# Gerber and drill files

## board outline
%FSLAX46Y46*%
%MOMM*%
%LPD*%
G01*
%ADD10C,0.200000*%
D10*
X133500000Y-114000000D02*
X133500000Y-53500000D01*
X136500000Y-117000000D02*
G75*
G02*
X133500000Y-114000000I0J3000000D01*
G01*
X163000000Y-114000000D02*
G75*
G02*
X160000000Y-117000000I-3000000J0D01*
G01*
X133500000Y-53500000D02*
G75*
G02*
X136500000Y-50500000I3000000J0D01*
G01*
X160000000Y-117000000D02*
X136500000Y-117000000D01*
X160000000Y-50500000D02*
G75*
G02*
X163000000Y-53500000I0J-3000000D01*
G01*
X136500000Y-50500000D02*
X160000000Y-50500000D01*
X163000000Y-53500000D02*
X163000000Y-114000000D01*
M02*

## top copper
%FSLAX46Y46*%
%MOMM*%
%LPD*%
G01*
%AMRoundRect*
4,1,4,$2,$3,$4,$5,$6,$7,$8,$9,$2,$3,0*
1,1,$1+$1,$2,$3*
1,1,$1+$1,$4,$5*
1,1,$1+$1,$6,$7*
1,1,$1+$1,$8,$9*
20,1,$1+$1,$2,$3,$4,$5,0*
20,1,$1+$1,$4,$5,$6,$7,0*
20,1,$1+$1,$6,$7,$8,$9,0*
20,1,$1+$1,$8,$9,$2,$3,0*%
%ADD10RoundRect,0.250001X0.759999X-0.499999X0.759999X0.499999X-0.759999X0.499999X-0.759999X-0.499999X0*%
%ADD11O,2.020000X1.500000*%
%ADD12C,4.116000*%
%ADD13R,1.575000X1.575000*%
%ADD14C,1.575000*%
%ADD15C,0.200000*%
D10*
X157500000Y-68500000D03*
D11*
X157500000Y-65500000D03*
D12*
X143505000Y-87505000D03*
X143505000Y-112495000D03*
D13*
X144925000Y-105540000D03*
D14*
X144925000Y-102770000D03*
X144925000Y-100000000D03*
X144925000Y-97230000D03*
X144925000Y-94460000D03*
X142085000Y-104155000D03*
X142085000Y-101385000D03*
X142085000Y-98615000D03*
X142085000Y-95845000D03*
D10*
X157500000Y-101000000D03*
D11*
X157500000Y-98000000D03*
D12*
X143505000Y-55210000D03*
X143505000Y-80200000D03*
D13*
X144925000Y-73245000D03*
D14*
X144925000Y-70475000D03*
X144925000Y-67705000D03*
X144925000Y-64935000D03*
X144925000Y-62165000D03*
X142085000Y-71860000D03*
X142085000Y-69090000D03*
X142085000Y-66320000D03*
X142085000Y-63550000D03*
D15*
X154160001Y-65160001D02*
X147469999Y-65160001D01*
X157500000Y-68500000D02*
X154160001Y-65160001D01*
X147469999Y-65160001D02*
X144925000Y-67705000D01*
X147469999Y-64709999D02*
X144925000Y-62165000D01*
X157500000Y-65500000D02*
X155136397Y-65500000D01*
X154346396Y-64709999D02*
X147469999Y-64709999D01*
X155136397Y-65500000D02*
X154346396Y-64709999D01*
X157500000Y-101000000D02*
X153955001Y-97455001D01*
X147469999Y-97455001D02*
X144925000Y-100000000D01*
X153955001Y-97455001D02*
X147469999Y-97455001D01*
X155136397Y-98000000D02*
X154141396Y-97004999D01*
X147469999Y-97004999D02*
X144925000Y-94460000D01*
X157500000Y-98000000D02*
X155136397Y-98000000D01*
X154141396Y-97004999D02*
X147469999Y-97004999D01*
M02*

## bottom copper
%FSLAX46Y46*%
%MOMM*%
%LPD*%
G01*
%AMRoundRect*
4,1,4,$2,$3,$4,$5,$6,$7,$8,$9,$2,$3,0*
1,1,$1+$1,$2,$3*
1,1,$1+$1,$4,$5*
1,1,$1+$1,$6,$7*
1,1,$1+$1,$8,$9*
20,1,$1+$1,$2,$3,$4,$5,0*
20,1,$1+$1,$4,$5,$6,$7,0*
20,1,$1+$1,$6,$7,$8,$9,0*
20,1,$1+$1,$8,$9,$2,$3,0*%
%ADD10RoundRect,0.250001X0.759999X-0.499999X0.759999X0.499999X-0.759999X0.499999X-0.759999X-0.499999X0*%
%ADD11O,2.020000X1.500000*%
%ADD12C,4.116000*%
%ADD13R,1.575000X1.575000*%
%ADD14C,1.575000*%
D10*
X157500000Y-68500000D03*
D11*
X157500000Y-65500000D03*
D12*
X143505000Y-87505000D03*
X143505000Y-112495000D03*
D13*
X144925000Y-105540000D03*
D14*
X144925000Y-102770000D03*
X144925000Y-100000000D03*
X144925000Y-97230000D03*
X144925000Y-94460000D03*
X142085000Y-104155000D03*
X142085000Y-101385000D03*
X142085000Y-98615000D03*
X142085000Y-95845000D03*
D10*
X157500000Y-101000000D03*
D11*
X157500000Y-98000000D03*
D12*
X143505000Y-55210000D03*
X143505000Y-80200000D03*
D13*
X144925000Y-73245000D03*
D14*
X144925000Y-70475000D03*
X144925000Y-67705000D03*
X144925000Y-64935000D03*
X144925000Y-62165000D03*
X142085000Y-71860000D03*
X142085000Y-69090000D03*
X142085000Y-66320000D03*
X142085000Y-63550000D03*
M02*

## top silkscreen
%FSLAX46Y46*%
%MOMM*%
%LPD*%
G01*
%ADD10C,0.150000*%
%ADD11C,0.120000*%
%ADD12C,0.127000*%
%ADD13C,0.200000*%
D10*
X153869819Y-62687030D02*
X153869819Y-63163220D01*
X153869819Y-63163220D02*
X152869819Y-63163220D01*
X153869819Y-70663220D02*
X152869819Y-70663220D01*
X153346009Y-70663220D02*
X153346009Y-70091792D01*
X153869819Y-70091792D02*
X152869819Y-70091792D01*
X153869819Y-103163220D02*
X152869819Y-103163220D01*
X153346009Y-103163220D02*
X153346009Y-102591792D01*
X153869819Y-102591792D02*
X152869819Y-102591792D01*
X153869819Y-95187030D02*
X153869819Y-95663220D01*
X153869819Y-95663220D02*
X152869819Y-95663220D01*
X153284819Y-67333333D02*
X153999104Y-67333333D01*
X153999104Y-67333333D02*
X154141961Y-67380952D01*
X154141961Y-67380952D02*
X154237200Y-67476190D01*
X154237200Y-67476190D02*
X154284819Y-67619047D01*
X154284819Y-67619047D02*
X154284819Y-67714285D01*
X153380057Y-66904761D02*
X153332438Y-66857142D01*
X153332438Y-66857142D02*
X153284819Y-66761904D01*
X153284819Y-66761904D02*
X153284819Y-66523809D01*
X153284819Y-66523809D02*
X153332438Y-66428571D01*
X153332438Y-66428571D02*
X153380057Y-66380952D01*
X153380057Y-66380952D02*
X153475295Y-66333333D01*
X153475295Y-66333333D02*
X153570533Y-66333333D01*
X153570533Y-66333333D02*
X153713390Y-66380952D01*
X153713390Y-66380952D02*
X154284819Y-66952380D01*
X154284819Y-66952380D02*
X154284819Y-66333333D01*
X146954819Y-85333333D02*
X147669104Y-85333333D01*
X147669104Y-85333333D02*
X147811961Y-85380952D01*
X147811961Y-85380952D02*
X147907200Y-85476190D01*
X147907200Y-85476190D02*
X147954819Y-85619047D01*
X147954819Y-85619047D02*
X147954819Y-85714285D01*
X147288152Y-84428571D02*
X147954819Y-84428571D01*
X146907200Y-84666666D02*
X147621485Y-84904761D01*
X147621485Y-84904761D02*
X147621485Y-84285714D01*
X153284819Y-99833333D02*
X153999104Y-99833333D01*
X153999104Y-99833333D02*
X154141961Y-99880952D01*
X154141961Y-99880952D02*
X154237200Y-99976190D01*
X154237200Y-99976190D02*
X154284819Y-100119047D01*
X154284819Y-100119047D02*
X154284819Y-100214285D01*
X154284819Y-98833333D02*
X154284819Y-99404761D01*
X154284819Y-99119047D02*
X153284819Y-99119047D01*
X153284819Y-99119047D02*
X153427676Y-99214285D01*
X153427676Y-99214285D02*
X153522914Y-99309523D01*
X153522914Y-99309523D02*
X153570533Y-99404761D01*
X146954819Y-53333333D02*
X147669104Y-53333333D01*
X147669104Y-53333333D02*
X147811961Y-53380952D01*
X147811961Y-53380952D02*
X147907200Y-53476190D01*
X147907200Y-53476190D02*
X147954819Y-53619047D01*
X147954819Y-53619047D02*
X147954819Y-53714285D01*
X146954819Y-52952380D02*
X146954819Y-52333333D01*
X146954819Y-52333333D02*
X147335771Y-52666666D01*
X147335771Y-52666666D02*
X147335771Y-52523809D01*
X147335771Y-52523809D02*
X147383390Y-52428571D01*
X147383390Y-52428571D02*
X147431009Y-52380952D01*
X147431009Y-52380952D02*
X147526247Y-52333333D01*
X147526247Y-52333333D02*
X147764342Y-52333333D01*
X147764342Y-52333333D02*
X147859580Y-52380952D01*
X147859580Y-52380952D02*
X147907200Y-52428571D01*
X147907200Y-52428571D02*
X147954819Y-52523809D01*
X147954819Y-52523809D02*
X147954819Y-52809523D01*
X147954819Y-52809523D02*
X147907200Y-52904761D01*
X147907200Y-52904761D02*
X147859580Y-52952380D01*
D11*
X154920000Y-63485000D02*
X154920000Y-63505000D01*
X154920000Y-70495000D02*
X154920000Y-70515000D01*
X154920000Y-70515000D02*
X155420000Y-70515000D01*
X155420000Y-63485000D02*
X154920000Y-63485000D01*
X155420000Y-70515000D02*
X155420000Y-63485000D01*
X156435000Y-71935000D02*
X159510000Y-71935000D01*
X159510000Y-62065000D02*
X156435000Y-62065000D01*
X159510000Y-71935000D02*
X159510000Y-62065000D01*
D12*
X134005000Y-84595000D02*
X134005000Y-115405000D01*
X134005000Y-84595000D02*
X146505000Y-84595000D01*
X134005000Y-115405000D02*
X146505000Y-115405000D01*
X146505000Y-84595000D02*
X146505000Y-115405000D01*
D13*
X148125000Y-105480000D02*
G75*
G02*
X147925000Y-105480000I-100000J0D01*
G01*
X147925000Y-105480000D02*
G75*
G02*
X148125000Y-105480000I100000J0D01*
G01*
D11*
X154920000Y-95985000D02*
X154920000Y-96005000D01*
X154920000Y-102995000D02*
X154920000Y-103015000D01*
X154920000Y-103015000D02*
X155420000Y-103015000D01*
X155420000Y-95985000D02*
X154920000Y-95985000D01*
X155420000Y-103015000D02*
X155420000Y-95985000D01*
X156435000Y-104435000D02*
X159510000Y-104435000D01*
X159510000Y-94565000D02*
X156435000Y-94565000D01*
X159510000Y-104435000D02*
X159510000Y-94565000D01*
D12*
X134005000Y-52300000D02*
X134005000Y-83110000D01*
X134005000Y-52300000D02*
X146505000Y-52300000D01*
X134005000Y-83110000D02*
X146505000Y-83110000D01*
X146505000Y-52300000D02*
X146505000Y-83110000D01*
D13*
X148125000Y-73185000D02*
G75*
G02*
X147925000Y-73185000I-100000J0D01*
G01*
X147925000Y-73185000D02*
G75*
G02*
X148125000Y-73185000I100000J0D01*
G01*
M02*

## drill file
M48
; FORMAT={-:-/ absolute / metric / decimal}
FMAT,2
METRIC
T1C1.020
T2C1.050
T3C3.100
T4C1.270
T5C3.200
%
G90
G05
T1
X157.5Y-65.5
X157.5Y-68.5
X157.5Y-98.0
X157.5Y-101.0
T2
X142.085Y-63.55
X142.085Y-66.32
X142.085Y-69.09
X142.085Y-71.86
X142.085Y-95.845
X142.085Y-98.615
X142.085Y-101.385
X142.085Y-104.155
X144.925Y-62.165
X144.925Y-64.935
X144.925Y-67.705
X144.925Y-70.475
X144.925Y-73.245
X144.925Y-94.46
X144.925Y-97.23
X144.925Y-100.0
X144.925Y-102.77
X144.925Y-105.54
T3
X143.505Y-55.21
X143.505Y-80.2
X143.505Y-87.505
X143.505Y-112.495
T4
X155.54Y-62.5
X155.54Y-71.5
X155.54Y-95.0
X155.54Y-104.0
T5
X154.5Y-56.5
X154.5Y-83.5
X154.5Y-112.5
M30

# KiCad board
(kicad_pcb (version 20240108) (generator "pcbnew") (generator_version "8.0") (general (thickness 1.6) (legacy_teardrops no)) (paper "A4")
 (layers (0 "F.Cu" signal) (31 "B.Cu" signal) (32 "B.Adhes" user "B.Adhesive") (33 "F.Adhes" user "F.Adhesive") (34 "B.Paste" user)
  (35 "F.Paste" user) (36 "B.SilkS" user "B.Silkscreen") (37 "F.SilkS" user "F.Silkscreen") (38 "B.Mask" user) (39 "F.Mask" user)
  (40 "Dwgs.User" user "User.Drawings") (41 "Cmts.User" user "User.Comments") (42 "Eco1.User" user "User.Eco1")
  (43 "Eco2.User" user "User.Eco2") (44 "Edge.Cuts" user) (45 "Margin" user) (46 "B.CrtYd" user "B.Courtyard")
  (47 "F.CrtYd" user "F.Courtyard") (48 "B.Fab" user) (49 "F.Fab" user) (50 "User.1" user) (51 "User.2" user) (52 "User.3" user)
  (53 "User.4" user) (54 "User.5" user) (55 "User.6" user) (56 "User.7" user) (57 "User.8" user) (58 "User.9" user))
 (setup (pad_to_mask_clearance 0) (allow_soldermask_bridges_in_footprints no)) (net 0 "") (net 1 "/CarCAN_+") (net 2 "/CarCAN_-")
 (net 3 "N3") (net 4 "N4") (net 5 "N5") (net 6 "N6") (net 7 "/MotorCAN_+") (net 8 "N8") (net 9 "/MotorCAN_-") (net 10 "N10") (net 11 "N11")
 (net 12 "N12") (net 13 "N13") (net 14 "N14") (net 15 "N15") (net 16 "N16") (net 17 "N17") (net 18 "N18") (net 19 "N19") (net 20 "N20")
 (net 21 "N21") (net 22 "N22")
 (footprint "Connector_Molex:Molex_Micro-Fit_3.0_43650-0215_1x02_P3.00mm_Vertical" (layer "F.Cu") (at 157.5 68.5 90)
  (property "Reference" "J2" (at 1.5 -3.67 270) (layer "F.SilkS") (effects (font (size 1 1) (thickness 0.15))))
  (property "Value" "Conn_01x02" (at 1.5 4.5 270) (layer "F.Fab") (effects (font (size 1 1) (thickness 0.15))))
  (fp_line (start 5.015 -2.58) (end 4.995 -2.58) (stroke (width 0.12) (type solid)) (layer "F.SilkS"))
  (fp_line (start -1.995 -2.58) (end -2.015 -2.58) (stroke (width 0.12) (type solid)) (layer "F.SilkS"))
  (fp_line (start -2.015 -2.58) (end -2.015 -2.08) (stroke (width 0.12) (type solid)) (layer "F.SilkS"))
  (fp_line (start 5.015 -2.08) (end 5.015 -2.58) (stroke (width 0.12) (type solid)) (layer "F.SilkS"))
  (fp_line (start -2.015 -2.08) (end 5.015 -2.08) (stroke (width 0.12) (type solid)) (layer "F.SilkS"))
  (fp_line (start -3.435 -1.065) (end -3.435 2.01) (stroke (width 0.12) (type solid)) (layer "F.SilkS"))
  (fp_line (start 6.435 2.01) (end 6.435 -1.065) (stroke (width 0.12) (type solid)) (layer "F.SilkS"))
  (fp_line (start -3.435 2.01) (end 6.435 2.01) (stroke (width 0.12) (type solid)) (layer "F.SilkS"))
  (pad "" np_thru_hole circle (at -3 -1.96 90) (size 1.27 1.27) (drill 1.27) (layers "*.Cu" "*.Mask"))
  (pad "" np_thru_hole circle (at 6 -1.96 90) (size 1.27 1.27) (drill 1.27) (layers "*.Cu" "*.Mask"))
  (pad "1" thru_hole roundrect (at 0 0 90) (size 1.5 2.02) (drill 1.02) (layers "*.Cu" "*.Mask") (remove_unused_layers no)
   (roundrect_rratio 0.166667) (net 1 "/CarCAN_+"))
  (pad "2" thru_hole oval (at 3 0 90) (size 1.5 2.02) (drill 1.02) (layers "*.Cu" "*.Mask") (remove_unused_layers no) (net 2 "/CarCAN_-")))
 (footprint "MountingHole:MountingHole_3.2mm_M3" (layer "F.Cu") (at 154.5 112.5)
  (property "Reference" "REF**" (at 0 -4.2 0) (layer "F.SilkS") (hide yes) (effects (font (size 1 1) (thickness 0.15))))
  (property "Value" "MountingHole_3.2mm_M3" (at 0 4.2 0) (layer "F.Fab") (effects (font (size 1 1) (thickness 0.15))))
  (pad "" np_thru_hole circle (at 0 0) (size 3.2 3.2) (drill 3.2) (layers "F&B.Cu" "*.Mask")))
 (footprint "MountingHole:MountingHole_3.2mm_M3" (layer "F.Cu") (at 154.5 56.5)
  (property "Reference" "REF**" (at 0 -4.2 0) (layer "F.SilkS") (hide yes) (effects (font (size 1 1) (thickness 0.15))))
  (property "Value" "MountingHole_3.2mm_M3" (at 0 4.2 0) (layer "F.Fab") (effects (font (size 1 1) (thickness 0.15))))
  (pad "" np_thru_hole circle (at 0 0) (size 3.2 3.2) (drill 3.2) (layers "*.Cu" "*.Mask")))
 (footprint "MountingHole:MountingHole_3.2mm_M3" (layer "F.Cu") (at 154.5 83.5)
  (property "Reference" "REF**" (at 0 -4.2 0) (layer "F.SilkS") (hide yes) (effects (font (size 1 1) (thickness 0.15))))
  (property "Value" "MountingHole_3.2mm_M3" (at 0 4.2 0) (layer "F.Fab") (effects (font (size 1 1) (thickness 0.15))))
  (pad "" np_thru_hole circle (at 0 0) (size 3.2 3.2) (drill 3.2) (layers "F&B.Cu" "*.Mask")))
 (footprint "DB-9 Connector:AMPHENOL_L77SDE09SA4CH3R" (layer "F.Cu") (at 143.505 100 -90)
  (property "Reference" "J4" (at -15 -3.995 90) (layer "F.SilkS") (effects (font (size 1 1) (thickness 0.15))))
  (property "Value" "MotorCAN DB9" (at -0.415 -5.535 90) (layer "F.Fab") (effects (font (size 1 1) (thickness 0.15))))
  (fp_line (start -15.405 9.5) (end 15.405 9.5) (stroke (width 0.127) (type solid)) (layer "F.SilkS"))
  (fp_line (start -15.405 9.5) (end -15.405 -3) (stroke (width 0.127) (type solid)) (layer "F.SilkS"))
  (fp_line (start 15.405 9.5) (end 15.405 -3) (stroke (width 0.127) (type solid)) (layer "F.SilkS"))
  (fp_line (start -15.405 -3) (end 15.405 -3) (stroke (width 0.127) (type solid)) (layer "F.SilkS"))
  (fp_circle (center 5.48 -4.52) (end 5.58 -4.52) (stroke (width 0.2) (type solid)) (fill none) (layer "F.SilkS"))
  (pad "0" thru_hole circle (at -12.495 0 270) (size 4.116 4.116) (drill 3.1) (layers "*.Cu" "*.Mask") (remove_unused_layers no)
   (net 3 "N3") (solder_mask_margin 0.102))
  (pad "0" thru_hole circle (at 12.495 0 270) (size 4.116 4.116) (drill 3.1) (layers "*.Cu" "*.Mask") (remove_unused_layers no) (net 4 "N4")
   (solder_mask_margin 0.102))
  (pad "1" thru_hole rect (at 5.54 -1.42 270) (size 1.575 1.575) (drill 1.05) (layers "*.Cu" "*.Mask") (remove_unused_layers no)
   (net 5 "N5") (solder_mask_margin 0.102))
  (pad "2" thru_hole circle (at 2.77 -1.42 270) (size 1.575 1.575) (drill 1.05) (layers "*.Cu" "*.Mask") (remove_unused_layers no)
   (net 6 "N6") (solder_mask_margin 0.102))
  (pad "3" thru_hole circle (at 0 -1.42 270) (size 1.575 1.575) (drill 1.05) (layers "*.Cu" "*.Mask") (remove_unused_layers no)
   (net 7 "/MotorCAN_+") (solder_mask_margin 0.102))
  (pad "4" thru_hole circle (at -2.77 -1.42 270) (size 1.575 1.575) (drill 1.05) (layers "*.Cu" "*.Mask") (remove_unused_layers no)
   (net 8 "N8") (solder_mask_margin 0.102))
  (pad "5" thru_hole circle (at -5.54 -1.42 270) (size 1.575 1.575) (drill 1.05) (layers "*.Cu" "*.Mask") (remove_unused_layers no)
   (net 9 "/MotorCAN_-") (solder_mask_margin 0.102))
  (pad "6" thru_hole circle (at 4.155 1.42 270) (size 1.575 1.575) (drill 1.05) (layers "*.Cu" "*.Mask") (remove_unused_layers no)
   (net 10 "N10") (solder_mask_margin 0.102))
  (pad "7" thru_hole circle (at 1.385 1.42 270) (size 1.575 1.575) (drill 1.05) (layers "*.Cu" "*.Mask") (remove_unused_layers no)
   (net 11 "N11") (solder_mask_margin 0.102))
  (pad "8" thru_hole circle (at -1.385 1.42 270) (size 1.575 1.575) (drill 1.05) (layers "*.Cu" "*.Mask") (remove_unused_layers no)
   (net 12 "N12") (solder_mask_margin 0.102))
  (pad "9" thru_hole circle (at -4.155 1.42 270) (size 1.575 1.575) (drill 1.05) (layers "*.Cu" "*.Mask") (remove_unused_layers no)
   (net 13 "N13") (solder_mask_margin 0.102)))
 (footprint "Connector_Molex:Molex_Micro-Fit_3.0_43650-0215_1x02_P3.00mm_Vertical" (layer "F.Cu") (at 157.5 101 90)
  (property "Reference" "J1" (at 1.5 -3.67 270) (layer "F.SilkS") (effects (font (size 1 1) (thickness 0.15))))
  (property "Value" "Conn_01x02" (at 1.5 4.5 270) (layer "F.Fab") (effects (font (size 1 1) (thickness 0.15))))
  (fp_line (start 5.015 -2.58) (end 4.995 -2.58) (stroke (width 0.12) (type solid)) (layer "F.SilkS"))
  (fp_line (start -1.995 -2.58) (end -2.015 -2.58) (stroke (width 0.12) (type solid)) (layer "F.SilkS"))
  (fp_line (start -2.015 -2.58) (end -2.015 -2.08) (stroke (width 0.12) (type solid)) (layer "F.SilkS"))
  (fp_line (start 5.015 -2.08) (end 5.015 -2.58) (stroke (width 0.12) (type solid)) (layer "F.SilkS"))
  (fp_line (start -2.015 -2.08) (end 5.015 -2.08) (stroke (width 0.12) (type solid)) (layer "F.SilkS"))
  (fp_line (start -3.435 -1.065) (end -3.435 2.01) (stroke (width 0.12) (type solid)) (layer "F.SilkS"))
  (fp_line (start 6.435 2.01) (end 6.435 -1.065) (stroke (width 0.12) (type solid)) (layer "F.SilkS"))
  (fp_line (start -3.435 2.01) (end 6.435 2.01) (stroke (width 0.12) (type solid)) (layer "F.SilkS"))
  (pad "" np_thru_hole circle (at -3 -1.96 90) (size 1.27 1.27) (drill 1.27) (layers "*.Cu" "*.Mask"))
  (pad "" np_thru_hole circle (at 6 -1.96 90) (size 1.27 1.27) (drill 1.27) (layers "*.Cu" "*.Mask"))
  (pad "1" thru_hole roundrect (at 0 0 90) (size 1.5 2.02) (drill 1.02) (layers "*.Cu" "*.Mask") (remove_unused_layers no)
   (roundrect_rratio 0.166667) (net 7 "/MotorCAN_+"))
  (pad "2" thru_hole oval (at 3 0 90) (size 1.5 2.02) (drill 1.02) (layers "*.Cu" "*.Mask") (remove_unused_layers no) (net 9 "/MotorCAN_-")))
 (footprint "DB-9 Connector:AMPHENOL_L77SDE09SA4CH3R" (layer "F.Cu") (at 143.505 67.705 -90)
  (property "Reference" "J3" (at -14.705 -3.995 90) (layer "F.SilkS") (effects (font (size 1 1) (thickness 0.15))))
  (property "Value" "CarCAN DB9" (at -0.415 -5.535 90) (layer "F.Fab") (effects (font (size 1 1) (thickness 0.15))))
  (fp_line (start -15.405 9.5) (end 15.405 9.5) (stroke (width 0.127) (type solid)) (layer "F.SilkS"))
  (fp_line (start -15.405 9.5) (end -15.405 -3) (stroke (width 0.127) (type solid)) (layer "F.SilkS"))
  (fp_line (start 15.405 9.5) (end 15.405 -3) (stroke (width 0.127) (type solid)) (layer "F.SilkS"))
  (fp_line (start -15.405 -3) (end 15.405 -3) (stroke (width 0.127) (type solid)) (layer "F.SilkS"))
  (fp_circle (center 5.48 -4.52) (end 5.58 -4.52) (stroke (width 0.2) (type solid)) (fill none) (layer "F.SilkS"))
  (pad "0" thru_hole circle (at -12.495 0 270) (size 4.116 4.116) (drill 3.1) (layers "*.Cu" "*.Mask") (remove_unused_layers no)
   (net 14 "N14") (solder_mask_margin 0.102))
  (pad "0" thru_hole circle (at 12.495 0 270) (size 4.116 4.116) (drill 3.1) (layers "*.Cu" "*.Mask") (remove_unused_layers no)
   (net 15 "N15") (solder_mask_margin 0.102))
  (pad "1" thru_hole rect (at 5.54 -1.42 270) (size 1.575 1.575) (drill 1.05) (layers "*.Cu" "*.Mask") (remove_unused_layers no)
   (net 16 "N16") (solder_mask_margin 0.102))
  (pad "2" thru_hole circle (at 2.77 -1.42 270) (size 1.575 1.575) (drill 1.05) (layers "*.Cu" "*.Mask") (remove_unused_layers no)
   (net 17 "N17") (solder_mask_margin 0.102))
  (pad "3" thru_hole circle (at 0 -1.42 270) (size 1.575 1.575) (drill 1.05) (layers "*.Cu" "*.Mask") (remove_unused_layers no)
   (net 1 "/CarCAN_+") (solder_mask_margin 0.102))
  (pad "4" thru_hole circle (at -2.77 -1.42 270) (size 1.575 1.575) (drill 1.05) (layers "*.Cu" "*.Mask") (remove_unused_layers no)
   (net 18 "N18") (solder_mask_margin 0.102))
  (pad "5" thru_hole circle (at -5.54 -1.42 270) (size 1.575 1.575) (drill 1.05) (layers "*.Cu" "*.Mask") (remove_unused_layers no)
   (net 2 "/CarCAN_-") (solder_mask_margin 0.102))
  (pad "6" thru_hole circle (at 4.155 1.42 270) (size 1.575 1.575) (drill 1.05) (layers "*.Cu" "*.Mask") (remove_unused_layers no)
   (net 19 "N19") (solder_mask_margin 0.102))
  (pad "7" thru_hole circle (at 1.385 1.42 270) (size 1.575 1.575) (drill 1.05) (layers "*.Cu" "*.Mask") (remove_unused_layers no)
   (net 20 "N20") (solder_mask_margin 0.102))
  (pad "8" thru_hole circle (at -1.385 1.42 270) (size 1.575 1.575) (drill 1.05) (layers "*.Cu" "*.Mask") (remove_unused_layers no)
   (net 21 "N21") (solder_mask_margin 0.102))
  (pad "9" thru_hole circle (at -4.155 1.42 270) (size 1.575 1.575) (drill 1.05) (layers "*.Cu" "*.Mask") (remove_unused_layers no)
   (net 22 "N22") (solder_mask_margin 0.102)))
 (gr_line (start 133.5 114) (end 133.5 53.5) (stroke (width 0.2) (type default)) (layer "Edge.Cuts"))
 (gr_arc (start 136.5 117) (mid 134.37868 116.12132) (end 133.5 114) (stroke (width 0.2) (type default)) (layer "Edge.Cuts"))
 (gr_arc (start 163 114) (mid 162.12132 116.12132) (end 160 117) (stroke (width 0.2) (type default)) (layer "Edge.Cuts"))
 (gr_arc (start 133.5 53.5) (mid 134.37868 51.37868) (end 136.5 50.5) (stroke (width 0.2) (type default)) (layer "Edge.Cuts"))
 (gr_line (start 160 117) (end 136.5 117) (stroke (width 0.2) (type default)) (layer "Edge.Cuts"))
 (gr_arc (start 160 50.5) (mid 162.12132 51.37868) (end 163 53.5) (stroke (width 0.2) (type default)) (layer "Edge.Cuts"))
 (gr_line (start 136.5 50.5) (end 160 50.5) (stroke (width 0.2) (type default)) (layer "Edge.Cuts"))
 (gr_line (start 163 53.5) (end 163 114) (stroke (width 0.2) (type default)) (layer "Edge.Cuts"))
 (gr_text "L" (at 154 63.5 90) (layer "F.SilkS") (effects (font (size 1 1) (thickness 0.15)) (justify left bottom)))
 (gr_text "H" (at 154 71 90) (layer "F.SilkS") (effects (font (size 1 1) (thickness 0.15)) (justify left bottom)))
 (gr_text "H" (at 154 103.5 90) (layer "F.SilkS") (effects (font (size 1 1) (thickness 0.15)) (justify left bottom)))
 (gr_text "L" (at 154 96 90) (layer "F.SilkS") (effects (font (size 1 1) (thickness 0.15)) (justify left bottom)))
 (segment (start 154.160001 65.160001) (end 147.469999 65.160001) (width 0.2) (layer "F.Cu") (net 1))
 (segment (start 157.5 68.5) (end 154.160001 65.160001) (width 0.2) (layer "F.Cu") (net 1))
 (segment (start 147.469999 65.160001) (end 144.925 67.705) (width 0.2) (layer "F.Cu") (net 1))
 (segment (start 147.469999 64.709999) (end 144.925 62.165) (width 0.2) (layer "F.Cu") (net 2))
 (segment (start 157.5 65.5) (end 155.136397 65.5) (width 0.2) (layer "F.Cu") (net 2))
 (segment (start 154.346396 64.709999) (end 147.469999 64.709999) (width 0.2) (layer "F.Cu") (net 2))
 (segment (start 155.136397 65.5) (end 154.346396 64.709999) (width 0.2) (layer "F.Cu") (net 2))
 (segment (start 157.5 101) (end 153.955001 97.455001) (width 0.2) (layer "F.Cu") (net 7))
 (segment (start 147.469999 97.455001) (end 144.925 100) (width 0.2) (layer "F.Cu") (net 7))
 (segment (start 153.955001 97.455001) (end 147.469999 97.455001) (width 0.2) (layer "F.Cu") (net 7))
 (segment (start 155.136397 98) (end 154.141396 97.004999) (width 0.2) (layer "F.Cu") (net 9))
 (segment (start 147.469999 97.004999) (end 144.925 94.46) (width 0.2) (layer "F.Cu") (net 9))
 (segment (start 157.5 98) (end 155.136397 98) (width 0.2) (layer "F.Cu") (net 9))
 (segment (start 154.141396 97.004999) (end 147.469999 97.004999) (width 0.2) (layer "F.Cu") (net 9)))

